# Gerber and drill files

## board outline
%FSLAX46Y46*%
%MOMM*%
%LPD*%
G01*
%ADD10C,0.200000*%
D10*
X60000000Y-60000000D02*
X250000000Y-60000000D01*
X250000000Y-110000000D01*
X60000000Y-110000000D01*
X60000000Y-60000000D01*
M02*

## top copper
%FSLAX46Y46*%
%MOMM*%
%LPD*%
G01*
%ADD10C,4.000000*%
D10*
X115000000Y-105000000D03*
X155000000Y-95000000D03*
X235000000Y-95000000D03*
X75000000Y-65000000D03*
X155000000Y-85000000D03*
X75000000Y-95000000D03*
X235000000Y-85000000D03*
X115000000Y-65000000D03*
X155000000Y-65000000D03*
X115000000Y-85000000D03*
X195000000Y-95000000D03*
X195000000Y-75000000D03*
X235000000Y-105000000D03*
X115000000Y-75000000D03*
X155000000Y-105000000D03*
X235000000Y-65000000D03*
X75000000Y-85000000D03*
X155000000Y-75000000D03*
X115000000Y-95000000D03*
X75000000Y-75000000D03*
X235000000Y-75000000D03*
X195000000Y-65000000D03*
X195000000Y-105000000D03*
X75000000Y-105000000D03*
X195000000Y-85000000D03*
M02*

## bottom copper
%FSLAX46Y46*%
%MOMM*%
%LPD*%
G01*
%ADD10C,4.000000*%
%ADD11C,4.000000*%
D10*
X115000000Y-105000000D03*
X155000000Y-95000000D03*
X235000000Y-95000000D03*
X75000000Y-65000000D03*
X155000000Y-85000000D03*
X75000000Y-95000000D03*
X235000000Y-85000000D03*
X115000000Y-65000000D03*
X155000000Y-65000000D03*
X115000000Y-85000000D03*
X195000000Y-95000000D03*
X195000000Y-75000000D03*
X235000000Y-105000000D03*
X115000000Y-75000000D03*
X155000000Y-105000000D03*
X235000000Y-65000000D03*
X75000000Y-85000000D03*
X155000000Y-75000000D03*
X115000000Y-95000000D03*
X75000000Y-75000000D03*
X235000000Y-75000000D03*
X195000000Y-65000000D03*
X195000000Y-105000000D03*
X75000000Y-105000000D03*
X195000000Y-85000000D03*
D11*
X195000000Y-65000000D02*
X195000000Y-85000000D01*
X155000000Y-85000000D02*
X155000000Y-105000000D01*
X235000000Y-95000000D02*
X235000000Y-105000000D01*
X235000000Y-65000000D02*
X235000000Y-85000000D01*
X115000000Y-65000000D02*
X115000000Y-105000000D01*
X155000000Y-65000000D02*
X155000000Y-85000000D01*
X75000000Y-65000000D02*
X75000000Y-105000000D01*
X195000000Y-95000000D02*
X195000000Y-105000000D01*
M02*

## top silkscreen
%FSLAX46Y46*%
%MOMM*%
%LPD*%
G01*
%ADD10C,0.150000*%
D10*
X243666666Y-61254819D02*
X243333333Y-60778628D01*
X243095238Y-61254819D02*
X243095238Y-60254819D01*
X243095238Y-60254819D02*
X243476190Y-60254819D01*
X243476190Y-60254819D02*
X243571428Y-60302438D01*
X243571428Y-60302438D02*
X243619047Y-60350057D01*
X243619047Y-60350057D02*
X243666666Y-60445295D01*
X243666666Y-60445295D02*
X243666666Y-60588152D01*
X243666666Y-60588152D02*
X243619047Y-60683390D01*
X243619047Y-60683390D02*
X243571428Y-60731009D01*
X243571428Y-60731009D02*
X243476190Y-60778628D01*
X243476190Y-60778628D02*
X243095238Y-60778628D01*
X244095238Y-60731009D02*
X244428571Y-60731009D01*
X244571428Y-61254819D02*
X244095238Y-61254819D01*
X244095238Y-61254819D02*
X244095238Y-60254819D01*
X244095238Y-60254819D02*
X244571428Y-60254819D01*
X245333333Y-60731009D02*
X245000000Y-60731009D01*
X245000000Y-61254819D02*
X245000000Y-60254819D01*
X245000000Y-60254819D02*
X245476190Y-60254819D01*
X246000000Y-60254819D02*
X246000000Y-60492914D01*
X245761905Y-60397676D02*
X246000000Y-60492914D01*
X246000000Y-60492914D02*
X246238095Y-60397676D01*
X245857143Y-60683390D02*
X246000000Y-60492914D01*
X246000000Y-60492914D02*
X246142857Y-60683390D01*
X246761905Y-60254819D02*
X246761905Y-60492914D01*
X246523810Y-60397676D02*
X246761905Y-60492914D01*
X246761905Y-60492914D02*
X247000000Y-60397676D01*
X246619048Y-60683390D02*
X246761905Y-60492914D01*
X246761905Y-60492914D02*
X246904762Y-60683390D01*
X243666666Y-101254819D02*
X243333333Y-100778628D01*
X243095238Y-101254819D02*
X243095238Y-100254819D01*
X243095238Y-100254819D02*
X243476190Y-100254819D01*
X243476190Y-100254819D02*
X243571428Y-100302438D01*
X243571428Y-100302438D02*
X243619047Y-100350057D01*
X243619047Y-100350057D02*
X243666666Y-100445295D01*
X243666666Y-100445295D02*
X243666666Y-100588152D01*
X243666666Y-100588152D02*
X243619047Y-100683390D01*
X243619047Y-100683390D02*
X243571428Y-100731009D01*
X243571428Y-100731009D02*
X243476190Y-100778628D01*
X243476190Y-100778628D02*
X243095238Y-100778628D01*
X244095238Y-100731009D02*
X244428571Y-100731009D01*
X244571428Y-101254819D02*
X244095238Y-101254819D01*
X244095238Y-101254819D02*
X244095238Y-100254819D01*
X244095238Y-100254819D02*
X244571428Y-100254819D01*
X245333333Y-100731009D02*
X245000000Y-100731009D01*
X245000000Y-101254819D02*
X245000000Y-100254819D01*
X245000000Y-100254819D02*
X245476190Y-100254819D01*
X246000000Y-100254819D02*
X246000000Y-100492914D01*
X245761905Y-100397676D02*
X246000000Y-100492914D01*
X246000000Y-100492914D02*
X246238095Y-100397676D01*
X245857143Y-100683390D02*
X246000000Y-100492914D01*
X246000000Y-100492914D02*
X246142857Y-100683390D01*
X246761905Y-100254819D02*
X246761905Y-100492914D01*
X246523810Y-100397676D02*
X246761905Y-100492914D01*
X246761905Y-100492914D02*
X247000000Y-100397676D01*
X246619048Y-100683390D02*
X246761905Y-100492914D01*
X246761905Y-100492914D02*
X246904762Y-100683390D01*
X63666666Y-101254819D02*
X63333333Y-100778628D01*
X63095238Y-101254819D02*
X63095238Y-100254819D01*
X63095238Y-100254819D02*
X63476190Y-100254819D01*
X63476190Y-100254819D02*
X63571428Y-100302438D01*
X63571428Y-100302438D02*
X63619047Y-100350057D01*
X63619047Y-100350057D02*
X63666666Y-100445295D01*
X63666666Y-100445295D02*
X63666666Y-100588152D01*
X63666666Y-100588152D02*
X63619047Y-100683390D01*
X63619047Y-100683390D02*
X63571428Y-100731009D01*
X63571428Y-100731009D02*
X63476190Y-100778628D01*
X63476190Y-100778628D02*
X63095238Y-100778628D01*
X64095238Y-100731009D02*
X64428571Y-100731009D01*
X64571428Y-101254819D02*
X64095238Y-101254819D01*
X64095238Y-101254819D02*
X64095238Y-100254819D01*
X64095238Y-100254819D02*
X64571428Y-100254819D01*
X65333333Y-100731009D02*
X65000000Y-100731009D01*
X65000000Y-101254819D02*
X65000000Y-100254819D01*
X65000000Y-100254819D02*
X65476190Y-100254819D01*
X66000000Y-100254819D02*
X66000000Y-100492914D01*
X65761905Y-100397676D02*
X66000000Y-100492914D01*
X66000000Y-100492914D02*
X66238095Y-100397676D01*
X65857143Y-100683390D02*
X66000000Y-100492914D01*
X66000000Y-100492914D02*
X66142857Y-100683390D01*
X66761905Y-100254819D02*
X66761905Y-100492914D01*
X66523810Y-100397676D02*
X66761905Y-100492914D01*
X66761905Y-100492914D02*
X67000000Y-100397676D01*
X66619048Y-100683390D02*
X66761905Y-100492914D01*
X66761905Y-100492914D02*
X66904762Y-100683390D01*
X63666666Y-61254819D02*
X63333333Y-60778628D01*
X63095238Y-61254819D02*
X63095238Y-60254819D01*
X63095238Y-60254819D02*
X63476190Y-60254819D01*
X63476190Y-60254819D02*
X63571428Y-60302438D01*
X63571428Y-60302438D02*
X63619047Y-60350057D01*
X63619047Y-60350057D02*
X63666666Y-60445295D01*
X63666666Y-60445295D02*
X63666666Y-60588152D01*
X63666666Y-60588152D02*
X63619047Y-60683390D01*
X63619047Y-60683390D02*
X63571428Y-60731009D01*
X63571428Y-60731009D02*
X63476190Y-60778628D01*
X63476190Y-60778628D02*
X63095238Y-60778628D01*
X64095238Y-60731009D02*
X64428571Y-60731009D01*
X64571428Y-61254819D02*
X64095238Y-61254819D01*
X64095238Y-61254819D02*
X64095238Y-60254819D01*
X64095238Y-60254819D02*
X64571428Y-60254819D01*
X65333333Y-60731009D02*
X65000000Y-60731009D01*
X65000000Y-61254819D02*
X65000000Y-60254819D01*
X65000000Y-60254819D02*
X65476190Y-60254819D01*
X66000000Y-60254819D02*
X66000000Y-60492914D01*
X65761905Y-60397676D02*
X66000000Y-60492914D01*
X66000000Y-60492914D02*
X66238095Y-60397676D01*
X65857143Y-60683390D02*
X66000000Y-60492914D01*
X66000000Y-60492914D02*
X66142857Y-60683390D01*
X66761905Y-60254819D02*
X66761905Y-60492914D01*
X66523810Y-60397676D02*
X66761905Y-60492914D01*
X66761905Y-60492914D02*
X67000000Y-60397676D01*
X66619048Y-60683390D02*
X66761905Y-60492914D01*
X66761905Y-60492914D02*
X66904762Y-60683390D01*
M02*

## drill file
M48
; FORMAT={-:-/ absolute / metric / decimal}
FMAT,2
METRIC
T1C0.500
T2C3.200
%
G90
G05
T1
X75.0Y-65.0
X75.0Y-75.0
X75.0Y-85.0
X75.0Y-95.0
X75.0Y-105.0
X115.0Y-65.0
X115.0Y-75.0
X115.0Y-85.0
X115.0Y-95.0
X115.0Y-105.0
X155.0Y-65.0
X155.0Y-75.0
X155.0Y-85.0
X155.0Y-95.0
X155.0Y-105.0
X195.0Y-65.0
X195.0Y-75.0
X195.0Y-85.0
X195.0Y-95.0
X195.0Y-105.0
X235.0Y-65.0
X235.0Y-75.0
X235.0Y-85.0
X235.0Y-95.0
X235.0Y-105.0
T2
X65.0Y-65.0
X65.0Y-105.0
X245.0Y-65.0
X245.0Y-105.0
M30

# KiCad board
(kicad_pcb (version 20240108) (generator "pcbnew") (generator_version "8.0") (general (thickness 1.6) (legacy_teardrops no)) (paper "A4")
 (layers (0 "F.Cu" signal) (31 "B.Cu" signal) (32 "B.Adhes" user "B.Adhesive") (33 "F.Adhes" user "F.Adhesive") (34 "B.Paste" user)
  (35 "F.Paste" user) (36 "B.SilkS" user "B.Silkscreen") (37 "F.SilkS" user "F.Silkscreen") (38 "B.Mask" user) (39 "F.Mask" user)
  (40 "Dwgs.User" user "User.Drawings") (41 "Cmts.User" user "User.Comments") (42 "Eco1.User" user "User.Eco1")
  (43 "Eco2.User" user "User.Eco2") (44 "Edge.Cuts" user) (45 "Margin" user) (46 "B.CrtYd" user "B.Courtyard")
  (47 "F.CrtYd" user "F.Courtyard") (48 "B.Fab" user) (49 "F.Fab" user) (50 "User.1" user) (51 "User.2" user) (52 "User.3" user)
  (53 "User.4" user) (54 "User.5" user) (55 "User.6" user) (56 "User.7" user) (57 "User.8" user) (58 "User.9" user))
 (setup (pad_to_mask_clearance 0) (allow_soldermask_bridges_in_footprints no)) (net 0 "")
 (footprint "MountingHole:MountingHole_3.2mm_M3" (layer "F.Cu") (at 245 65)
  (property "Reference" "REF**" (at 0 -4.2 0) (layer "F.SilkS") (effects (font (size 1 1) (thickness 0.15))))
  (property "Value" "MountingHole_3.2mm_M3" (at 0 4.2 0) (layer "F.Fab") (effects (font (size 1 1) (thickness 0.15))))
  (pad "" np_thru_hole circle (at 0 0) (size 3.2 3.2) (drill 3.2) (layers "F&B.Cu" "*.Mask")))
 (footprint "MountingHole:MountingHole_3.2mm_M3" (layer "F.Cu") (at 245 105)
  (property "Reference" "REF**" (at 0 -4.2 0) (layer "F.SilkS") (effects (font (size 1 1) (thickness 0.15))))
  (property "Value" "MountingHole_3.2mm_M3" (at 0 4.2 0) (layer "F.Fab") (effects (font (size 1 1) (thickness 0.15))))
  (pad "" np_thru_hole circle (at 0 0) (size 3.2 3.2) (drill 3.2) (layers "F&B.Cu" "*.Mask")))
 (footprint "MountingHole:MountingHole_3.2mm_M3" (layer "F.Cu") (at 65 105)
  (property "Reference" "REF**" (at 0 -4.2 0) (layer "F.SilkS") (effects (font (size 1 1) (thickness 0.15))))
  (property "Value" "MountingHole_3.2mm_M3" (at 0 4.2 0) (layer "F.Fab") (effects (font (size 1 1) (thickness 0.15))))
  (pad "" np_thru_hole circle (at 0 0) (size 3.2 3.2) (drill 3.2) (layers "F&B.Cu" "*.Mask")))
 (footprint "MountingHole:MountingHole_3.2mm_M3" (layer "F.Cu") (at 65 65)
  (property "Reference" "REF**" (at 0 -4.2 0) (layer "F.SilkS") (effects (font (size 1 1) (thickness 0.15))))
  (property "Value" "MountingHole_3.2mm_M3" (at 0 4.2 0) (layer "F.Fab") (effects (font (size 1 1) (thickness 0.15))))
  (pad "" np_thru_hole circle (at 0 0) (size 3.2 3.2) (drill 3.2) (layers "*.Cu" "*.Mask")))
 (gr_rect (start 60 60) (end 250 110) (stroke (width 0.2) (type default)) (fill none) (layer "Edge.Cuts"))
 (via (at 115 105) (size 4) (drill 0.5) (layers "F.Cu" "B.Cu") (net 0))
 (via (at 155 95) (size 4) (drill 0.5) (layers "F.Cu" "B.Cu") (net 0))
 (via (at 235 95) (size 4) (drill 0.5) (layers "F.Cu" "B.Cu") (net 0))
 (via (at 75 65) (size 4) (drill 0.5) (layers "F.Cu" "B.Cu") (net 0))
 (via (at 155 85) (size 4) (drill 0.5) (layers "F.Cu" "B.Cu") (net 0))
 (via (at 75 95) (size 4) (drill 0.5) (layers "F.Cu" "B.Cu") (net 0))
 (via (at 235 85) (size 4) (drill 0.5) (layers "F.Cu" "B.Cu") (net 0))
 (via (at 115 65) (size 4) (drill 0.5) (layers "F.Cu" "B.Cu") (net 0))
 (via (at 155 65) (size 4) (drill 0.5) (layers "F.Cu" "B.Cu") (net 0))
 (via (at 115 85) (size 4) (drill 0.5) (layers "F.Cu" "B.Cu") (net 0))
 (via (at 195 95) (size 4) (drill 0.5) (layers "F.Cu" "B.Cu") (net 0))
 (via (at 195 75) (size 4) (drill 0.5) (layers "F.Cu" "B.Cu") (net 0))
 (via (at 235 105) (size 4) (drill 0.5) (layers "F.Cu" "B.Cu") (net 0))
 (via (at 115 75) (size 4) (drill 0.5) (layers "F.Cu" "B.Cu") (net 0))
 (via (at 155 105) (size 4) (drill 0.5) (layers "F.Cu" "B.Cu") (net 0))
 (via (at 235 65) (size 4) (drill 0.5) (layers "F.Cu" "B.Cu") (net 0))
 (via (at 75 85) (size 4) (drill 0.5) (layers "F.Cu" "B.Cu") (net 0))
 (via (at 155 75) (size 4) (drill 0.5) (layers "F.Cu" "B.Cu") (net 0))
 (via (at 115 95) (size 4) (drill 0.5) (layers "F.Cu" "B.Cu") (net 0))
 (via (at 75 75) (size 4) (drill 0.5) (layers "F.Cu" "B.Cu") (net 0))
 (via (at 235 75) (size 4) (drill 0.5) (layers "F.Cu" "B.Cu") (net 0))
 (via (at 195 65) (size 4) (drill 0.5) (layers "F.Cu" "B.Cu") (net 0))
 (via (at 195 105) (size 4) (drill 0.5) (layers "F.Cu" "B.Cu") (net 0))
 (via (at 75 105) (size 4) (drill 0.5) (layers "F.Cu" "B.Cu") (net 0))
 (via (at 195 85) (size 4) (drill 0.5) (layers "F.Cu" "B.Cu") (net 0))
 (segment (start 195 65) (end 195 85) (width 4) (layer "B.Cu") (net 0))
 (segment (start 155 85) (end 155 105) (width 4) (layer "B.Cu") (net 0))
 (segment (start 235 95) (end 235 105) (width 4) (layer "B.Cu") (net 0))
 (segment (start 235 65) (end 235 85) (width 4) (layer "B.Cu") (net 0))
 (segment (start 115 65) (end 115 105) (width 4) (layer "B.Cu") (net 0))
 (segment (start 155 65) (end 155 85) (width 4) (layer "B.Cu") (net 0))
 (segment (start 75 65) (end 75 105) (width 4) (layer "B.Cu") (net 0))
 (segment (start 195 95) (end 195 105) (width 4) (layer "B.Cu") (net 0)))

